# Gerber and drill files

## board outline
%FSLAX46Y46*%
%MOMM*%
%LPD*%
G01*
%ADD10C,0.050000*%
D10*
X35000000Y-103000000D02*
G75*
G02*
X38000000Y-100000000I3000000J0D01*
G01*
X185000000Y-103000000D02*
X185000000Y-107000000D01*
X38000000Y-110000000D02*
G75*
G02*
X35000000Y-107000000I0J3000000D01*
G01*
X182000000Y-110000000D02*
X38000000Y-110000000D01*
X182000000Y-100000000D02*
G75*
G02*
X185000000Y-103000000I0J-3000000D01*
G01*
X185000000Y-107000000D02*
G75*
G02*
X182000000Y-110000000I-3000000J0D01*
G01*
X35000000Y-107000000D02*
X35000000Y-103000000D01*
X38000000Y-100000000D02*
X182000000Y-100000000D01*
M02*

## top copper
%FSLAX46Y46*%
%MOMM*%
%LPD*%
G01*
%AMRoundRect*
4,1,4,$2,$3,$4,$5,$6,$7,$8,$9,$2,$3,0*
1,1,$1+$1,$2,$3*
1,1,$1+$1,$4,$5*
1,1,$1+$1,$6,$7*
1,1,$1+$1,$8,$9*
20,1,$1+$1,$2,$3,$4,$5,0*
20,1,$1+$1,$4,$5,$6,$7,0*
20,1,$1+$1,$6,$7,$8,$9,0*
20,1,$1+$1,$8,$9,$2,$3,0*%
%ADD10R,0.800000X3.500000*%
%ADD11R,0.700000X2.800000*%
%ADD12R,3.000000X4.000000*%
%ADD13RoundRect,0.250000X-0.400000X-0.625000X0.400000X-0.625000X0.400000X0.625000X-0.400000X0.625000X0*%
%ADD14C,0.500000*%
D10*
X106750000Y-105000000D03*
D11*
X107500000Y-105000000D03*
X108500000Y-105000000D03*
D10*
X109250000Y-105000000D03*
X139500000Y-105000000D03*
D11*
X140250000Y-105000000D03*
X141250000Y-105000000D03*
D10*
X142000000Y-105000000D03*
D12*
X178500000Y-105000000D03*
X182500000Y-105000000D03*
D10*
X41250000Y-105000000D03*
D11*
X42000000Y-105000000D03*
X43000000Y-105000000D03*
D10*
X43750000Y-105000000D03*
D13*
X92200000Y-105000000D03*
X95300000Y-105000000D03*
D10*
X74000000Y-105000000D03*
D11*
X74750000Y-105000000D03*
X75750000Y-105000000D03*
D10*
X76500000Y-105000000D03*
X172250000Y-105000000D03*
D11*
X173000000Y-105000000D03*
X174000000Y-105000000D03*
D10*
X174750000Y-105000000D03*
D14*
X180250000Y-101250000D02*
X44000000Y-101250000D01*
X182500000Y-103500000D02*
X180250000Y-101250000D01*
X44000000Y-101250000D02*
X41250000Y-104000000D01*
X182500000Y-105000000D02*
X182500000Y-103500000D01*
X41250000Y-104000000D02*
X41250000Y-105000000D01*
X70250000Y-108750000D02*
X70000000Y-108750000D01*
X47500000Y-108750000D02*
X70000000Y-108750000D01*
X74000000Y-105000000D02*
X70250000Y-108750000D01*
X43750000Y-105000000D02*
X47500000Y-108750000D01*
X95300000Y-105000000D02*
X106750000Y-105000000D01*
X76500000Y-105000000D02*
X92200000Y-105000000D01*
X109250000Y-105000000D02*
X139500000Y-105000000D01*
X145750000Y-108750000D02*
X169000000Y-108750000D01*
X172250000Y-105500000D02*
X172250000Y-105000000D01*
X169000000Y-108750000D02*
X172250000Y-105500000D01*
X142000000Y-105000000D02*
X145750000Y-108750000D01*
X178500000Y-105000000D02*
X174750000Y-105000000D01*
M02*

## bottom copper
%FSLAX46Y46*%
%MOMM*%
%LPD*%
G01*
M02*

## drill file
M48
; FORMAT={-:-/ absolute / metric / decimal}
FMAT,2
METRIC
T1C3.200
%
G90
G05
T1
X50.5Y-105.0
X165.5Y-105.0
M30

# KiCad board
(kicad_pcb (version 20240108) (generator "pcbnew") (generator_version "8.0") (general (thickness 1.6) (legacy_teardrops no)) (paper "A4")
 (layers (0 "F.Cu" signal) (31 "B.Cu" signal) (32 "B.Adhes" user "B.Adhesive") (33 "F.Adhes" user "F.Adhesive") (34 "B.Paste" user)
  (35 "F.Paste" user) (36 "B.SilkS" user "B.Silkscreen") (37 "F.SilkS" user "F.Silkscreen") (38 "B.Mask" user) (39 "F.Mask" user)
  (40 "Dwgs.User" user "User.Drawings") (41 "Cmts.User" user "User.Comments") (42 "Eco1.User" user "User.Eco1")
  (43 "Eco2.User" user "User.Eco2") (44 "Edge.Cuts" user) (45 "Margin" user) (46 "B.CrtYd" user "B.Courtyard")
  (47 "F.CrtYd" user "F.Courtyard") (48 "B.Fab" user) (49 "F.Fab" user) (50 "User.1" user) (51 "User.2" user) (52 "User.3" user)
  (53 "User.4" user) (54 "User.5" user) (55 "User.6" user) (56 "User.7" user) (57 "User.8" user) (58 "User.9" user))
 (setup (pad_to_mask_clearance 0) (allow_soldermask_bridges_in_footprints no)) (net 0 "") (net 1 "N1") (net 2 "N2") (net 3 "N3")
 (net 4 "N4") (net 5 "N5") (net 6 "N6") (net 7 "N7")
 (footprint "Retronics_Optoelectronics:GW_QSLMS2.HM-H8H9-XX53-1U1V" (layer "F.Cu") (at 108 105 90)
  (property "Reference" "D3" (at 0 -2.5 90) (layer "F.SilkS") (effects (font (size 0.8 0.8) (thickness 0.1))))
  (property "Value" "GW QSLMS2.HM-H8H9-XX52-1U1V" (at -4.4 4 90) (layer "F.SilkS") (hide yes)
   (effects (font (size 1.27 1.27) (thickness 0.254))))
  (pad "1" smd rect (at 0 -1.25 180) (size 0.8 3.5) (layers "F.Cu" "F.Paste" "F.Mask") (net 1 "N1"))
  (pad "1" smd rect (at 0 -0.5 180) (size 0.7 2.8) (layers "F.Cu" "F.Paste" "F.Mask") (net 1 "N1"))
  (pad "2" smd rect (at 0 0.5 180) (size 0.7 2.8) (layers "F.Cu" "F.Paste" "F.Mask") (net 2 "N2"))
  (pad "2" smd rect (at 0 1.25 180) (size 0.8 3.5) (layers "F.Cu" "F.Paste" "F.Mask") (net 2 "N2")))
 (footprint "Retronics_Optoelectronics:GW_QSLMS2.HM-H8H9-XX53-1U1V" (layer "F.Cu") (at 140.75 105 90)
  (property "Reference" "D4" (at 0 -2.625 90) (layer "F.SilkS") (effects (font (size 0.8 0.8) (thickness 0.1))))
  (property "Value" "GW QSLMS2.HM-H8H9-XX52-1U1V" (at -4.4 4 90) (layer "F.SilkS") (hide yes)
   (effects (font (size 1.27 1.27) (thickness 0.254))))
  (pad "1" smd rect (at 0 -1.25 180) (size 0.8 3.5) (layers "F.Cu" "F.Paste" "F.Mask") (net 2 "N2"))
  (pad "1" smd rect (at 0 -0.5 180) (size 0.7 2.8) (layers "F.Cu" "F.Paste" "F.Mask") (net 2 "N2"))
  (pad "2" smd rect (at 0 0.5 180) (size 0.7 2.8) (layers "F.Cu" "F.Paste" "F.Mask") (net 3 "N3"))
  (pad "2" smd rect (at 0 1.25 180) (size 0.8 3.5) (layers "F.Cu" "F.Paste" "F.Mask") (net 3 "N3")))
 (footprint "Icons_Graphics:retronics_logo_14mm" (layer "F.Cu") (at 125.503328 101.75)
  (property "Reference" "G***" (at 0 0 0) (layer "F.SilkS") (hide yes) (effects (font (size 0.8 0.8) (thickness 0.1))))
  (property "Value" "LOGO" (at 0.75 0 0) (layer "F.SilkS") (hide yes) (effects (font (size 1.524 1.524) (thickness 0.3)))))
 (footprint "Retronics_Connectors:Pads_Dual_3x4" (layer "F.Cu") (at 178.5 105)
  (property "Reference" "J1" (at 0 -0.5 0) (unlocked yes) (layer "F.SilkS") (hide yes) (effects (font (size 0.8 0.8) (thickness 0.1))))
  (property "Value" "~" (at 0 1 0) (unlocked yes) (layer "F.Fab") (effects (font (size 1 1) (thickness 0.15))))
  (pad "1" smd rect (at 0 0 180) (size 3 4) (layers "F.Cu" "F.Paste" "F.Mask") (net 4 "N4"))
  (pad "2" smd rect (at 4 0 180) (size 3 4) (layers "F.Cu" "F.Paste" "F.Mask") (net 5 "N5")))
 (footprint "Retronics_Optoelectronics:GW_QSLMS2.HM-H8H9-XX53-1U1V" (layer "F.Cu") (at 42.5 105 90)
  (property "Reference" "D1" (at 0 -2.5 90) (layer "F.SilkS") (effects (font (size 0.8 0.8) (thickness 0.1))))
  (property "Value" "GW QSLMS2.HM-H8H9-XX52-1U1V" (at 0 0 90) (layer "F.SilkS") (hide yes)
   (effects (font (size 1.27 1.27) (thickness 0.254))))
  (pad "1" smd rect (at 0 -1.25 180) (size 0.8 3.5) (layers "F.Cu" "F.Paste" "F.Mask") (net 5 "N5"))
  (pad "1" smd rect (at 0 -0.5 180) (size 0.7 2.8) (layers "F.Cu" "F.Paste" "F.Mask") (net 5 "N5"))
  (pad "2" smd rect (at 0 0.5 180) (size 0.7 2.8) (layers "F.Cu" "F.Paste" "F.Mask") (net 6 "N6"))
  (pad "2" smd rect (at 0 1.25 180) (size 0.8 3.5) (layers "F.Cu" "F.Paste" "F.Mask") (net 6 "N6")))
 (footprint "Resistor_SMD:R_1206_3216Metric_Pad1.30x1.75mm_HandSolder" (layer "F.Cu") (at 93.75 105)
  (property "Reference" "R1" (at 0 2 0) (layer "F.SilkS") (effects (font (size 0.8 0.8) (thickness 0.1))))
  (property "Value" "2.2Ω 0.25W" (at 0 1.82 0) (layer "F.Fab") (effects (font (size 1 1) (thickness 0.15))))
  (pad "1" smd roundrect (at -1.55 0) (size 1.3 1.75) (layers "F.Cu" "F.Paste" "F.Mask") (roundrect_rratio 0.192308) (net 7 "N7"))
  (pad "2" smd roundrect (at 1.55 0) (size 1.3 1.75) (layers "F.Cu" "F.Paste" "F.Mask") (roundrect_rratio 0.192308) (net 1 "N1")))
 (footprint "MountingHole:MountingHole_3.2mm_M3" (layer "F.Cu") (at 165.5 105)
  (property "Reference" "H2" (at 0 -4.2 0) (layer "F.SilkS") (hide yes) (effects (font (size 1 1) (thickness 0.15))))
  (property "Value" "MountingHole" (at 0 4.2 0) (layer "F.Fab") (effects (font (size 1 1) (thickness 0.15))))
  (pad "" np_thru_hole circle (at 0 0) (size 3.2 3.2) (drill 3.2) (layers "*.Cu" "*.Mask")))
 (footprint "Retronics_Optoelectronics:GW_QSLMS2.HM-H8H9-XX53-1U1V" (layer "F.Cu") (at 75.25 105 90)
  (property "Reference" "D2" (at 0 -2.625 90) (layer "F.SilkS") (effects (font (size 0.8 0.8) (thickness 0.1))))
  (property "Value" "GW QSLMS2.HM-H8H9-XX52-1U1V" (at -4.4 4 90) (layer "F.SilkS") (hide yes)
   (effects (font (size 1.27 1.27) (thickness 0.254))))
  (pad "1" smd rect (at 0 -1.25 180) (size 0.8 3.5) (layers "F.Cu" "F.Paste" "F.Mask") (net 6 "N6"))
  (pad "1" smd rect (at 0 -0.5 180) (size 0.7 2.8) (layers "F.Cu" "F.Paste" "F.Mask") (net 6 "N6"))
  (pad "2" smd rect (at 0 0.5 180) (size 0.7 2.8) (layers "F.Cu" "F.Paste" "F.Mask") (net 7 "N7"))
  (pad "2" smd rect (at 0 1.25 180) (size 0.8 3.5) (layers "F.Cu" "F.Paste" "F.Mask") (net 7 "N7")))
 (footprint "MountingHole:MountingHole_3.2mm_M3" (layer "F.Cu") (at 50.5 105)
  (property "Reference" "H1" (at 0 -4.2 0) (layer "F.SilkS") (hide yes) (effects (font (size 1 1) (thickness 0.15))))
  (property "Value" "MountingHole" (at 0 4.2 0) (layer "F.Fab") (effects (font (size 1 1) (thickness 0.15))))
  (pad "" np_thru_hole circle (at 0 0) (size 3.2 3.2) (drill 3.2) (layers "*.Cu" "*.Mask")))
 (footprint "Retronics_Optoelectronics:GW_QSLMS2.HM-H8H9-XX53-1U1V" (layer "F.Cu") (at 173.5 105 90)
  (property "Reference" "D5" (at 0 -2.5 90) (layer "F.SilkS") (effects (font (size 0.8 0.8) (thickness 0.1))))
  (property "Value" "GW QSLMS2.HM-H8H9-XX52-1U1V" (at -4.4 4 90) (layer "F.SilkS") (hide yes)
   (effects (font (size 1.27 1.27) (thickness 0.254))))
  (pad "1" smd rect (at 0 -1.25 180) (size 0.8 3.5) (layers "F.Cu" "F.Paste" "F.Mask") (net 3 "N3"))
  (pad "1" smd rect (at 0 -0.5 180) (size 0.7 2.8) (layers "F.Cu" "F.Paste" "F.Mask") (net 3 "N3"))
  (pad "2" smd rect (at 0 0.5 180) (size 0.7 2.8) (layers "F.Cu" "F.Paste" "F.Mask") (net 4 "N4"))
  (pad "2" smd rect (at 0 1.25 180) (size 0.8 3.5) (layers "F.Cu" "F.Paste" "F.Mask") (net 4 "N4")))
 (gr_arc (start 35 103) (mid 35.87868 100.87868) (end 38 100) (stroke (width 0.05) (type default)) (layer "Edge.Cuts"))
 (gr_line (start 185 103) (end 185 107) (stroke (width 0.05) (type default)) (layer "Edge.Cuts"))
 (gr_arc (start 38 110) (mid 35.87868 109.12132) (end 35 107) (stroke (width 0.05) (type default)) (layer "Edge.Cuts"))
 (gr_line (start 182 110) (end 38 110) (stroke (width 0.05) (type default)) (layer "Edge.Cuts"))
 (gr_arc (start 182 100) (mid 184.12132 100.87868) (end 185 103) (stroke (width 0.05) (type default)) (layer "Edge.Cuts"))
 (gr_arc (start 185 107) (mid 184.12132 109.12132) (end 182 110) (stroke (width 0.05) (type default)) (layer "Edge.Cuts"))
 (gr_line (start 35 107) (end 35 103) (stroke (width 0.05) (type default)) (layer "Edge.Cuts"))
 (gr_line (start 38 100) (end 182 100) (stroke (width 0.05) (type default)) (layer "Edge.Cuts"))
 (segment (start 180.25 101.25) (end 44 101.25) (width 0.5) (layer "F.Cu") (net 5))
 (segment (start 182.5 103.5) (end 180.25 101.25) (width 0.5) (layer "F.Cu") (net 5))
 (segment (start 44 101.25) (end 41.25 104) (width 0.5) (layer "F.Cu") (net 5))
 (segment (start 182.5 105) (end 182.5 103.5) (width 0.5) (layer "F.Cu") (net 5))
 (segment (start 41.25 104) (end 41.25 105) (width 0.5) (layer "F.Cu") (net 5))
 (segment (start 70.25 108.75) (end 70 108.75) (width 0.5) (layer "F.Cu") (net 6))
 (segment (start 47.5 108.75) (end 70 108.75) (width 0.5) (layer "F.Cu") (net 6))
 (segment (start 74 105) (end 70.25 108.75) (width 0.5) (layer "F.Cu") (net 6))
 (segment (start 43.75 105) (end 47.5 108.75) (width 0.5) (layer "F.Cu") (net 6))
 (segment (start 95.3 105) (end 106.75 105) (width 0.5) (layer "F.Cu") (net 1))
 (segment (start 76.5 105) (end 92.2 105) (width 0.5) (layer "F.Cu") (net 7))
 (segment (start 109.25 105) (end 139.5 105) (width 0.5) (layer "F.Cu") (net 2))
 (segment (start 145.75 108.75) (end 169 108.75) (width 0.5) (layer "F.Cu") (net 3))
 (segment (start 172.25 105.5) (end 172.25 105) (width 0.5) (layer "F.Cu") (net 3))
 (segment (start 169 108.75) (end 172.25 105.5) (width 0.5) (layer "F.Cu") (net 3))
 (segment (start 142 105) (end 145.75 108.75) (width 0.5) (layer "F.Cu") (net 3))
 (segment (start 178.5 105) (end 174.75 105) (width 0.5) (layer "F.Cu") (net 4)))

